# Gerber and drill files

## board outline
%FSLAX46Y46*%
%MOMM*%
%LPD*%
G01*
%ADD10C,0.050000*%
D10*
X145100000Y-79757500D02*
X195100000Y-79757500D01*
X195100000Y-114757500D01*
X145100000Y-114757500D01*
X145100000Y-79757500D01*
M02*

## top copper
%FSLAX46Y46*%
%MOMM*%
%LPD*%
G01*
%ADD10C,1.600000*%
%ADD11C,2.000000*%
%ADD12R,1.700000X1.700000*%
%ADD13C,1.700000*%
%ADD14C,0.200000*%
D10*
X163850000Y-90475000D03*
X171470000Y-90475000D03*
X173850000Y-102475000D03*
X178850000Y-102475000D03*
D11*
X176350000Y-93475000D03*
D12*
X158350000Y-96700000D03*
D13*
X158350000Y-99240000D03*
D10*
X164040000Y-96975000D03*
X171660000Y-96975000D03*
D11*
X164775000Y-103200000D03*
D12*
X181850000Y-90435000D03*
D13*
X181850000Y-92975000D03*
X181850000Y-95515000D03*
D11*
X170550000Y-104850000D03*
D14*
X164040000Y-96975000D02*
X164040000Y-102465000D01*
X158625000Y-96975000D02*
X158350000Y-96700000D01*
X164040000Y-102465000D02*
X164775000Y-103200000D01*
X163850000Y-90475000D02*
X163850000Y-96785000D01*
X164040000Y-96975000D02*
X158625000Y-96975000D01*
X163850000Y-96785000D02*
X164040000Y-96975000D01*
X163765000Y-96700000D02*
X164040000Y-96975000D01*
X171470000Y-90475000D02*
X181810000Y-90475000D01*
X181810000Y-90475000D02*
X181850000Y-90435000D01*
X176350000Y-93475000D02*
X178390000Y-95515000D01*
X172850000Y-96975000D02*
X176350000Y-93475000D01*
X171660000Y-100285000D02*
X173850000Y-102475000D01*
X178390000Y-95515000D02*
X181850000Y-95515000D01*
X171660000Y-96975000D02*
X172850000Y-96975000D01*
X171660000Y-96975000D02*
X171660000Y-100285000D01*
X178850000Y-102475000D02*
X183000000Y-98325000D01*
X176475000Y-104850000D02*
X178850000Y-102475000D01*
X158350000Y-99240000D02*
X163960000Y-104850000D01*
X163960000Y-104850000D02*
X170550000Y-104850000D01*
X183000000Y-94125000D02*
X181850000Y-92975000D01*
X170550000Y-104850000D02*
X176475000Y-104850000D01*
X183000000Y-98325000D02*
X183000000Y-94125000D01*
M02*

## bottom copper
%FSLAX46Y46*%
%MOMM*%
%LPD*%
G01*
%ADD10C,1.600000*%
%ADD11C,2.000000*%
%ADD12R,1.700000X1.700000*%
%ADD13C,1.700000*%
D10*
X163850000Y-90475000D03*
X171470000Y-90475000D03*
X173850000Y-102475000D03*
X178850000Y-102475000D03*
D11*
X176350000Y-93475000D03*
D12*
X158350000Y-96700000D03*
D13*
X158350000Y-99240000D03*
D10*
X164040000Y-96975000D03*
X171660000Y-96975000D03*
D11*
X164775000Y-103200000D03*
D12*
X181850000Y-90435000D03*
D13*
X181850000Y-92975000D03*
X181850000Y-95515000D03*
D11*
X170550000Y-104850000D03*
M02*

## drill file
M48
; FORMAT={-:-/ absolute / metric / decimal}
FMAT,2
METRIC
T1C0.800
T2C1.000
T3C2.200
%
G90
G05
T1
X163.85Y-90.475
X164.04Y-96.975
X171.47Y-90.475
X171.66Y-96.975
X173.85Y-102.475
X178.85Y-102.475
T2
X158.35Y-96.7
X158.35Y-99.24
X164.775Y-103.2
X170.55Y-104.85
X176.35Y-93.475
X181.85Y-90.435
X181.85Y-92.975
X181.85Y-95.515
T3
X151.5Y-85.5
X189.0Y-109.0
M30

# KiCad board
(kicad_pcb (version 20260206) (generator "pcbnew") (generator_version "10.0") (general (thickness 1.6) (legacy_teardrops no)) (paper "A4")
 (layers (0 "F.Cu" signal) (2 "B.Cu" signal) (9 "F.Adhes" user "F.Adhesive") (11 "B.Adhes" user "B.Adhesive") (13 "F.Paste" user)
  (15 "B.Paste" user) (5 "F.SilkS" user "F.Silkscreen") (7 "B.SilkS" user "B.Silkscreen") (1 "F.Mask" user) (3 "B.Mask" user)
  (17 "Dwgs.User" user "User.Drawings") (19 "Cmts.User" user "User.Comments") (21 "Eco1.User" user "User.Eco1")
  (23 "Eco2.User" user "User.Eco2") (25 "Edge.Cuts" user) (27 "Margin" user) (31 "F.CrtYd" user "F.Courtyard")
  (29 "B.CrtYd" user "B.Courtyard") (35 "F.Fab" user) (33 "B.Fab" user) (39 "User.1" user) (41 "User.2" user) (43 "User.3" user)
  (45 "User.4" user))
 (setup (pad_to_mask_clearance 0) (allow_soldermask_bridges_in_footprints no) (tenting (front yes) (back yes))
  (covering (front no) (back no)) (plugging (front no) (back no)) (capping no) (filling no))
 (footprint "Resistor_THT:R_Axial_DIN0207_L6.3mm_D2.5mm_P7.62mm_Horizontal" (layer "F.Cu") (at 163.85 90.475)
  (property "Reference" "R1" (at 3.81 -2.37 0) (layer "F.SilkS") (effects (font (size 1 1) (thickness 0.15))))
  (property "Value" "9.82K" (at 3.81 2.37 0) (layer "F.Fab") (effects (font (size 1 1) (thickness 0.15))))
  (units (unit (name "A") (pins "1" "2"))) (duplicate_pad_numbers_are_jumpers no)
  (pad "1" thru_hole circle (at 0 0) (size 1.6 1.6) (drill 0.8) (layers "*.Cu" "*.Mask") (remove_unused_layers no) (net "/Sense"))
  (pad "2" thru_hole circle (at 7.62 0) (size 1.6 1.6) (drill 0.8) (layers "*.Cu" "*.Mask") (remove_unused_layers no) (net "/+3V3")))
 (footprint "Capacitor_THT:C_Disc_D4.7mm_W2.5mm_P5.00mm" (layer "F.Cu") (at 173.85 102.475)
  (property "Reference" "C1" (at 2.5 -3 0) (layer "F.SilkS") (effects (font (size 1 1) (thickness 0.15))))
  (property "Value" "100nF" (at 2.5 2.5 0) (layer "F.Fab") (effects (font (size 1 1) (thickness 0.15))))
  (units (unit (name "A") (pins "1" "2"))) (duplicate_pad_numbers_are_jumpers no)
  (pad "1" thru_hole circle (at 0 0) (size 1.6 1.6) (drill 0.8) (layers "*.Cu" "*.Mask") (remove_unused_layers no) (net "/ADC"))
  (pad "2" thru_hole circle (at 5 0) (size 1.6 1.6) (drill 0.8) (layers "*.Cu" "*.Mask") (remove_unused_layers no) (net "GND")))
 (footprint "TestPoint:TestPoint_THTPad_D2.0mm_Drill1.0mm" (layer "F.Cu") (at 176.35 93.475)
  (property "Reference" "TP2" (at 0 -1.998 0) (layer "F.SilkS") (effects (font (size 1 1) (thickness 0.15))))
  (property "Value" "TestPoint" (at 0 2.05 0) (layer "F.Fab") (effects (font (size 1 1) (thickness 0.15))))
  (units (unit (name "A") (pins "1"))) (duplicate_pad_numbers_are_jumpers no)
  (pad "1" thru_hole circle (at 0 0) (size 2 2) (drill 1) (layers "*.Cu" "*.Mask") (remove_unused_layers no) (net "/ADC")))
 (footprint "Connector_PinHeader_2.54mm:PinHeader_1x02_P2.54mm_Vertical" (layer "F.Cu") (at 158.35 96.7)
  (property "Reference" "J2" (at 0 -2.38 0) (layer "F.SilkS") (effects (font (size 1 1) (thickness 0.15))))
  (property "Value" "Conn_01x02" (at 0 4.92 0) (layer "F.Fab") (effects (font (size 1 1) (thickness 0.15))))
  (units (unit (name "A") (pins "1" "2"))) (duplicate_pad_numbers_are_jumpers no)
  (pad "1" thru_hole rect (at 0 0) (size 1.7 1.7) (drill 1) (layers "*.Cu" "*.Mask") (remove_unused_layers no) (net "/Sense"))
  (pad "2" thru_hole circle (at 0 2.54) (size 1.7 1.7) (drill 1) (layers "*.Cu" "*.Mask") (remove_unused_layers no) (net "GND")))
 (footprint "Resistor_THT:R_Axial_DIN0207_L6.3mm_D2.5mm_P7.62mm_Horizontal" (layer "F.Cu") (at 164.04 96.975)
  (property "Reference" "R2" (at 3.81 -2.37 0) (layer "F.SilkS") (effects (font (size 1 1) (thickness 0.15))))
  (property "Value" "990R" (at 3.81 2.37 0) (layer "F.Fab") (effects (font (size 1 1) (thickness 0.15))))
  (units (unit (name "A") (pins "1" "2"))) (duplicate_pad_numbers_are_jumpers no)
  (pad "1" thru_hole circle (at 0 0) (size 1.6 1.6) (drill 0.8) (layers "*.Cu" "*.Mask") (remove_unused_layers no) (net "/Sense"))
  (pad "2" thru_hole circle (at 7.62 0) (size 1.6 1.6) (drill 0.8) (layers "*.Cu" "*.Mask") (remove_unused_layers no) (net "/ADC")))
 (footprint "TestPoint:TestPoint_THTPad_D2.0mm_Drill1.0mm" (layer "F.Cu") (at 164.775 103.2)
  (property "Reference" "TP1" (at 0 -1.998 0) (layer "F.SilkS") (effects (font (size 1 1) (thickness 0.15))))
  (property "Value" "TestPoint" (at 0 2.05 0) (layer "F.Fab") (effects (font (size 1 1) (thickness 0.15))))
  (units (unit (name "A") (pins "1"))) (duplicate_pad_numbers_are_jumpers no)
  (pad "1" thru_hole circle (at 0 0) (size 2 2) (drill 1) (layers "*.Cu" "*.Mask") (remove_unused_layers no) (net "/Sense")))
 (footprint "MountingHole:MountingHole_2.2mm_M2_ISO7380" (layer "F.Cu") (at 151.5 85.5)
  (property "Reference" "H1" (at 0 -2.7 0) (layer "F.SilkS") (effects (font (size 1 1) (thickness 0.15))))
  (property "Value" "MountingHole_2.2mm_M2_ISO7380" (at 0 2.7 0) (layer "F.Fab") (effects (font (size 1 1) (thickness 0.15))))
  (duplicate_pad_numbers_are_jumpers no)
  (pad "" np_thru_hole circle (at 0 0) (size 2.2 2.2) (drill 2.2) (layers "*.Cu" "*.Mask")))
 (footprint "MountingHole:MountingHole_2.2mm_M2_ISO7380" (layer "F.Cu") (at 189 109)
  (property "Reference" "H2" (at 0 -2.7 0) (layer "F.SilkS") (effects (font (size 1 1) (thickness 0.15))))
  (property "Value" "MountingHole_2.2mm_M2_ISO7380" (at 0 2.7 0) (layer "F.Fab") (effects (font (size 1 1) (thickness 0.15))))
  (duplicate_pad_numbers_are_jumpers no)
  (pad "" np_thru_hole circle (at 0 0) (size 2.2 2.2) (drill 2.2) (layers "*.Cu" "*.Mask")))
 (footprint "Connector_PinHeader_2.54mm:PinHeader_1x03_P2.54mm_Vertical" (layer "F.Cu") (at 181.85 90.435)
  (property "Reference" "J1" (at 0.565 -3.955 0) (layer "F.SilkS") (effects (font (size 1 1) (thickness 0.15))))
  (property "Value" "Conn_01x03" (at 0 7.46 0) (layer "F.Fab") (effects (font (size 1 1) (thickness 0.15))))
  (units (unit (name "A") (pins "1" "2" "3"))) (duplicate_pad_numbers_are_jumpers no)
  (pad "1" thru_hole rect (at 0 0) (size 1.7 1.7) (drill 1) (layers "*.Cu" "*.Mask") (remove_unused_layers no) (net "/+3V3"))
  (pad "2" thru_hole circle (at 0 2.54) (size 1.7 1.7) (drill 1) (layers "*.Cu" "*.Mask") (remove_unused_layers no) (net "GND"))
  (pad "3" thru_hole circle (at 0 5.08) (size 1.7 1.7) (drill 1) (layers "*.Cu" "*.Mask") (remove_unused_layers no) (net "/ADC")))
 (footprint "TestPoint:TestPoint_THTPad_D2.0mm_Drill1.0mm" (layer "F.Cu") (at 170.55 104.85)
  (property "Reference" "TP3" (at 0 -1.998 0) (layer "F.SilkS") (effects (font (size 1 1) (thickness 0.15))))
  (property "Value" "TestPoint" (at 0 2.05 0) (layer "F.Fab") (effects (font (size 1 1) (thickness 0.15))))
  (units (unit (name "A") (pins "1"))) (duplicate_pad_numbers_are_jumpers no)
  (pad "1" thru_hole circle (at 0 0) (size 2 2) (drill 1) (layers "*.Cu" "*.Mask") (remove_unused_layers no) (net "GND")))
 (gr_rect (start 145.1 79.7575) (end 195.1 114.7575) (stroke (width 0.05) (type solid)) (fill no) (layer "Edge.Cuts"))
 (segment (start 164.04 96.975) (end 164.04 102.465) (width 0.2) (layer "F.Cu") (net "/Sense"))
 (segment (start 158.625 96.975) (end 158.35 96.7) (width 0.2) (layer "F.Cu") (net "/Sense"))
 (segment (start 164.04 102.465) (end 164.775 103.2) (width 0.2) (layer "F.Cu") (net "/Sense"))
 (segment (start 163.85 90.475) (end 163.85 96.785) (width 0.2) (layer "F.Cu") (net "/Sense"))
 (segment (start 164.04 96.975) (end 158.625 96.975) (width 0.2) (layer "F.Cu") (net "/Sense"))
 (segment (start 163.85 96.785) (end 164.04 96.975) (width 0.2) (layer "F.Cu") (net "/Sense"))
 (segment (start 163.765 96.7) (end 164.04 96.975) (width 0.2) (layer "F.Cu") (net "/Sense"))
 (segment (start 171.47 90.475) (end 181.81 90.475) (width 0.2) (layer "F.Cu") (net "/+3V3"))
 (segment (start 181.81 90.475) (end 181.85 90.435) (width 0.2) (layer "F.Cu") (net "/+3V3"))
 (segment (start 176.35 93.475) (end 178.39 95.515) (width 0.2) (layer "F.Cu") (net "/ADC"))
 (segment (start 172.85 96.975) (end 176.35 93.475) (width 0.2) (layer "F.Cu") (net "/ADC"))
 (segment (start 171.66 100.285) (end 173.85 102.475) (width 0.2) (layer "F.Cu") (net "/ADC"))
 (segment (start 178.39 95.515) (end 181.85 95.515) (width 0.2) (layer "F.Cu") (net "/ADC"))
 (segment (start 171.66 96.975) (end 172.85 96.975) (width 0.2) (layer "F.Cu") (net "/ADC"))
 (segment (start 171.66 96.975) (end 171.66 100.285) (width 0.2) (layer "F.Cu") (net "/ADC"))
 (segment (start 178.85 102.475) (end 183 98.325) (width 0.2) (layer "F.Cu") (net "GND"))
 (segment (start 176.475 104.85) (end 178.85 102.475) (width 0.2) (layer "F.Cu") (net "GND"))
 (segment (start 158.35 99.24) (end 163.96 104.85) (width 0.2) (layer "F.Cu") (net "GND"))
 (segment (start 163.96 104.85) (end 170.55 104.85) (width 0.2) (layer "F.Cu") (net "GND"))
 (segment (start 183 94.125) (end 181.85 92.975) (width 0.2) (layer "F.Cu") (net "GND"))
 (segment (start 170.55 104.85) (end 176.475 104.85) (width 0.2) (layer "F.Cu") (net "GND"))
 (segment (start 183 98.325) (end 183 94.125) (width 0.2) (layer "F.Cu") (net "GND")))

